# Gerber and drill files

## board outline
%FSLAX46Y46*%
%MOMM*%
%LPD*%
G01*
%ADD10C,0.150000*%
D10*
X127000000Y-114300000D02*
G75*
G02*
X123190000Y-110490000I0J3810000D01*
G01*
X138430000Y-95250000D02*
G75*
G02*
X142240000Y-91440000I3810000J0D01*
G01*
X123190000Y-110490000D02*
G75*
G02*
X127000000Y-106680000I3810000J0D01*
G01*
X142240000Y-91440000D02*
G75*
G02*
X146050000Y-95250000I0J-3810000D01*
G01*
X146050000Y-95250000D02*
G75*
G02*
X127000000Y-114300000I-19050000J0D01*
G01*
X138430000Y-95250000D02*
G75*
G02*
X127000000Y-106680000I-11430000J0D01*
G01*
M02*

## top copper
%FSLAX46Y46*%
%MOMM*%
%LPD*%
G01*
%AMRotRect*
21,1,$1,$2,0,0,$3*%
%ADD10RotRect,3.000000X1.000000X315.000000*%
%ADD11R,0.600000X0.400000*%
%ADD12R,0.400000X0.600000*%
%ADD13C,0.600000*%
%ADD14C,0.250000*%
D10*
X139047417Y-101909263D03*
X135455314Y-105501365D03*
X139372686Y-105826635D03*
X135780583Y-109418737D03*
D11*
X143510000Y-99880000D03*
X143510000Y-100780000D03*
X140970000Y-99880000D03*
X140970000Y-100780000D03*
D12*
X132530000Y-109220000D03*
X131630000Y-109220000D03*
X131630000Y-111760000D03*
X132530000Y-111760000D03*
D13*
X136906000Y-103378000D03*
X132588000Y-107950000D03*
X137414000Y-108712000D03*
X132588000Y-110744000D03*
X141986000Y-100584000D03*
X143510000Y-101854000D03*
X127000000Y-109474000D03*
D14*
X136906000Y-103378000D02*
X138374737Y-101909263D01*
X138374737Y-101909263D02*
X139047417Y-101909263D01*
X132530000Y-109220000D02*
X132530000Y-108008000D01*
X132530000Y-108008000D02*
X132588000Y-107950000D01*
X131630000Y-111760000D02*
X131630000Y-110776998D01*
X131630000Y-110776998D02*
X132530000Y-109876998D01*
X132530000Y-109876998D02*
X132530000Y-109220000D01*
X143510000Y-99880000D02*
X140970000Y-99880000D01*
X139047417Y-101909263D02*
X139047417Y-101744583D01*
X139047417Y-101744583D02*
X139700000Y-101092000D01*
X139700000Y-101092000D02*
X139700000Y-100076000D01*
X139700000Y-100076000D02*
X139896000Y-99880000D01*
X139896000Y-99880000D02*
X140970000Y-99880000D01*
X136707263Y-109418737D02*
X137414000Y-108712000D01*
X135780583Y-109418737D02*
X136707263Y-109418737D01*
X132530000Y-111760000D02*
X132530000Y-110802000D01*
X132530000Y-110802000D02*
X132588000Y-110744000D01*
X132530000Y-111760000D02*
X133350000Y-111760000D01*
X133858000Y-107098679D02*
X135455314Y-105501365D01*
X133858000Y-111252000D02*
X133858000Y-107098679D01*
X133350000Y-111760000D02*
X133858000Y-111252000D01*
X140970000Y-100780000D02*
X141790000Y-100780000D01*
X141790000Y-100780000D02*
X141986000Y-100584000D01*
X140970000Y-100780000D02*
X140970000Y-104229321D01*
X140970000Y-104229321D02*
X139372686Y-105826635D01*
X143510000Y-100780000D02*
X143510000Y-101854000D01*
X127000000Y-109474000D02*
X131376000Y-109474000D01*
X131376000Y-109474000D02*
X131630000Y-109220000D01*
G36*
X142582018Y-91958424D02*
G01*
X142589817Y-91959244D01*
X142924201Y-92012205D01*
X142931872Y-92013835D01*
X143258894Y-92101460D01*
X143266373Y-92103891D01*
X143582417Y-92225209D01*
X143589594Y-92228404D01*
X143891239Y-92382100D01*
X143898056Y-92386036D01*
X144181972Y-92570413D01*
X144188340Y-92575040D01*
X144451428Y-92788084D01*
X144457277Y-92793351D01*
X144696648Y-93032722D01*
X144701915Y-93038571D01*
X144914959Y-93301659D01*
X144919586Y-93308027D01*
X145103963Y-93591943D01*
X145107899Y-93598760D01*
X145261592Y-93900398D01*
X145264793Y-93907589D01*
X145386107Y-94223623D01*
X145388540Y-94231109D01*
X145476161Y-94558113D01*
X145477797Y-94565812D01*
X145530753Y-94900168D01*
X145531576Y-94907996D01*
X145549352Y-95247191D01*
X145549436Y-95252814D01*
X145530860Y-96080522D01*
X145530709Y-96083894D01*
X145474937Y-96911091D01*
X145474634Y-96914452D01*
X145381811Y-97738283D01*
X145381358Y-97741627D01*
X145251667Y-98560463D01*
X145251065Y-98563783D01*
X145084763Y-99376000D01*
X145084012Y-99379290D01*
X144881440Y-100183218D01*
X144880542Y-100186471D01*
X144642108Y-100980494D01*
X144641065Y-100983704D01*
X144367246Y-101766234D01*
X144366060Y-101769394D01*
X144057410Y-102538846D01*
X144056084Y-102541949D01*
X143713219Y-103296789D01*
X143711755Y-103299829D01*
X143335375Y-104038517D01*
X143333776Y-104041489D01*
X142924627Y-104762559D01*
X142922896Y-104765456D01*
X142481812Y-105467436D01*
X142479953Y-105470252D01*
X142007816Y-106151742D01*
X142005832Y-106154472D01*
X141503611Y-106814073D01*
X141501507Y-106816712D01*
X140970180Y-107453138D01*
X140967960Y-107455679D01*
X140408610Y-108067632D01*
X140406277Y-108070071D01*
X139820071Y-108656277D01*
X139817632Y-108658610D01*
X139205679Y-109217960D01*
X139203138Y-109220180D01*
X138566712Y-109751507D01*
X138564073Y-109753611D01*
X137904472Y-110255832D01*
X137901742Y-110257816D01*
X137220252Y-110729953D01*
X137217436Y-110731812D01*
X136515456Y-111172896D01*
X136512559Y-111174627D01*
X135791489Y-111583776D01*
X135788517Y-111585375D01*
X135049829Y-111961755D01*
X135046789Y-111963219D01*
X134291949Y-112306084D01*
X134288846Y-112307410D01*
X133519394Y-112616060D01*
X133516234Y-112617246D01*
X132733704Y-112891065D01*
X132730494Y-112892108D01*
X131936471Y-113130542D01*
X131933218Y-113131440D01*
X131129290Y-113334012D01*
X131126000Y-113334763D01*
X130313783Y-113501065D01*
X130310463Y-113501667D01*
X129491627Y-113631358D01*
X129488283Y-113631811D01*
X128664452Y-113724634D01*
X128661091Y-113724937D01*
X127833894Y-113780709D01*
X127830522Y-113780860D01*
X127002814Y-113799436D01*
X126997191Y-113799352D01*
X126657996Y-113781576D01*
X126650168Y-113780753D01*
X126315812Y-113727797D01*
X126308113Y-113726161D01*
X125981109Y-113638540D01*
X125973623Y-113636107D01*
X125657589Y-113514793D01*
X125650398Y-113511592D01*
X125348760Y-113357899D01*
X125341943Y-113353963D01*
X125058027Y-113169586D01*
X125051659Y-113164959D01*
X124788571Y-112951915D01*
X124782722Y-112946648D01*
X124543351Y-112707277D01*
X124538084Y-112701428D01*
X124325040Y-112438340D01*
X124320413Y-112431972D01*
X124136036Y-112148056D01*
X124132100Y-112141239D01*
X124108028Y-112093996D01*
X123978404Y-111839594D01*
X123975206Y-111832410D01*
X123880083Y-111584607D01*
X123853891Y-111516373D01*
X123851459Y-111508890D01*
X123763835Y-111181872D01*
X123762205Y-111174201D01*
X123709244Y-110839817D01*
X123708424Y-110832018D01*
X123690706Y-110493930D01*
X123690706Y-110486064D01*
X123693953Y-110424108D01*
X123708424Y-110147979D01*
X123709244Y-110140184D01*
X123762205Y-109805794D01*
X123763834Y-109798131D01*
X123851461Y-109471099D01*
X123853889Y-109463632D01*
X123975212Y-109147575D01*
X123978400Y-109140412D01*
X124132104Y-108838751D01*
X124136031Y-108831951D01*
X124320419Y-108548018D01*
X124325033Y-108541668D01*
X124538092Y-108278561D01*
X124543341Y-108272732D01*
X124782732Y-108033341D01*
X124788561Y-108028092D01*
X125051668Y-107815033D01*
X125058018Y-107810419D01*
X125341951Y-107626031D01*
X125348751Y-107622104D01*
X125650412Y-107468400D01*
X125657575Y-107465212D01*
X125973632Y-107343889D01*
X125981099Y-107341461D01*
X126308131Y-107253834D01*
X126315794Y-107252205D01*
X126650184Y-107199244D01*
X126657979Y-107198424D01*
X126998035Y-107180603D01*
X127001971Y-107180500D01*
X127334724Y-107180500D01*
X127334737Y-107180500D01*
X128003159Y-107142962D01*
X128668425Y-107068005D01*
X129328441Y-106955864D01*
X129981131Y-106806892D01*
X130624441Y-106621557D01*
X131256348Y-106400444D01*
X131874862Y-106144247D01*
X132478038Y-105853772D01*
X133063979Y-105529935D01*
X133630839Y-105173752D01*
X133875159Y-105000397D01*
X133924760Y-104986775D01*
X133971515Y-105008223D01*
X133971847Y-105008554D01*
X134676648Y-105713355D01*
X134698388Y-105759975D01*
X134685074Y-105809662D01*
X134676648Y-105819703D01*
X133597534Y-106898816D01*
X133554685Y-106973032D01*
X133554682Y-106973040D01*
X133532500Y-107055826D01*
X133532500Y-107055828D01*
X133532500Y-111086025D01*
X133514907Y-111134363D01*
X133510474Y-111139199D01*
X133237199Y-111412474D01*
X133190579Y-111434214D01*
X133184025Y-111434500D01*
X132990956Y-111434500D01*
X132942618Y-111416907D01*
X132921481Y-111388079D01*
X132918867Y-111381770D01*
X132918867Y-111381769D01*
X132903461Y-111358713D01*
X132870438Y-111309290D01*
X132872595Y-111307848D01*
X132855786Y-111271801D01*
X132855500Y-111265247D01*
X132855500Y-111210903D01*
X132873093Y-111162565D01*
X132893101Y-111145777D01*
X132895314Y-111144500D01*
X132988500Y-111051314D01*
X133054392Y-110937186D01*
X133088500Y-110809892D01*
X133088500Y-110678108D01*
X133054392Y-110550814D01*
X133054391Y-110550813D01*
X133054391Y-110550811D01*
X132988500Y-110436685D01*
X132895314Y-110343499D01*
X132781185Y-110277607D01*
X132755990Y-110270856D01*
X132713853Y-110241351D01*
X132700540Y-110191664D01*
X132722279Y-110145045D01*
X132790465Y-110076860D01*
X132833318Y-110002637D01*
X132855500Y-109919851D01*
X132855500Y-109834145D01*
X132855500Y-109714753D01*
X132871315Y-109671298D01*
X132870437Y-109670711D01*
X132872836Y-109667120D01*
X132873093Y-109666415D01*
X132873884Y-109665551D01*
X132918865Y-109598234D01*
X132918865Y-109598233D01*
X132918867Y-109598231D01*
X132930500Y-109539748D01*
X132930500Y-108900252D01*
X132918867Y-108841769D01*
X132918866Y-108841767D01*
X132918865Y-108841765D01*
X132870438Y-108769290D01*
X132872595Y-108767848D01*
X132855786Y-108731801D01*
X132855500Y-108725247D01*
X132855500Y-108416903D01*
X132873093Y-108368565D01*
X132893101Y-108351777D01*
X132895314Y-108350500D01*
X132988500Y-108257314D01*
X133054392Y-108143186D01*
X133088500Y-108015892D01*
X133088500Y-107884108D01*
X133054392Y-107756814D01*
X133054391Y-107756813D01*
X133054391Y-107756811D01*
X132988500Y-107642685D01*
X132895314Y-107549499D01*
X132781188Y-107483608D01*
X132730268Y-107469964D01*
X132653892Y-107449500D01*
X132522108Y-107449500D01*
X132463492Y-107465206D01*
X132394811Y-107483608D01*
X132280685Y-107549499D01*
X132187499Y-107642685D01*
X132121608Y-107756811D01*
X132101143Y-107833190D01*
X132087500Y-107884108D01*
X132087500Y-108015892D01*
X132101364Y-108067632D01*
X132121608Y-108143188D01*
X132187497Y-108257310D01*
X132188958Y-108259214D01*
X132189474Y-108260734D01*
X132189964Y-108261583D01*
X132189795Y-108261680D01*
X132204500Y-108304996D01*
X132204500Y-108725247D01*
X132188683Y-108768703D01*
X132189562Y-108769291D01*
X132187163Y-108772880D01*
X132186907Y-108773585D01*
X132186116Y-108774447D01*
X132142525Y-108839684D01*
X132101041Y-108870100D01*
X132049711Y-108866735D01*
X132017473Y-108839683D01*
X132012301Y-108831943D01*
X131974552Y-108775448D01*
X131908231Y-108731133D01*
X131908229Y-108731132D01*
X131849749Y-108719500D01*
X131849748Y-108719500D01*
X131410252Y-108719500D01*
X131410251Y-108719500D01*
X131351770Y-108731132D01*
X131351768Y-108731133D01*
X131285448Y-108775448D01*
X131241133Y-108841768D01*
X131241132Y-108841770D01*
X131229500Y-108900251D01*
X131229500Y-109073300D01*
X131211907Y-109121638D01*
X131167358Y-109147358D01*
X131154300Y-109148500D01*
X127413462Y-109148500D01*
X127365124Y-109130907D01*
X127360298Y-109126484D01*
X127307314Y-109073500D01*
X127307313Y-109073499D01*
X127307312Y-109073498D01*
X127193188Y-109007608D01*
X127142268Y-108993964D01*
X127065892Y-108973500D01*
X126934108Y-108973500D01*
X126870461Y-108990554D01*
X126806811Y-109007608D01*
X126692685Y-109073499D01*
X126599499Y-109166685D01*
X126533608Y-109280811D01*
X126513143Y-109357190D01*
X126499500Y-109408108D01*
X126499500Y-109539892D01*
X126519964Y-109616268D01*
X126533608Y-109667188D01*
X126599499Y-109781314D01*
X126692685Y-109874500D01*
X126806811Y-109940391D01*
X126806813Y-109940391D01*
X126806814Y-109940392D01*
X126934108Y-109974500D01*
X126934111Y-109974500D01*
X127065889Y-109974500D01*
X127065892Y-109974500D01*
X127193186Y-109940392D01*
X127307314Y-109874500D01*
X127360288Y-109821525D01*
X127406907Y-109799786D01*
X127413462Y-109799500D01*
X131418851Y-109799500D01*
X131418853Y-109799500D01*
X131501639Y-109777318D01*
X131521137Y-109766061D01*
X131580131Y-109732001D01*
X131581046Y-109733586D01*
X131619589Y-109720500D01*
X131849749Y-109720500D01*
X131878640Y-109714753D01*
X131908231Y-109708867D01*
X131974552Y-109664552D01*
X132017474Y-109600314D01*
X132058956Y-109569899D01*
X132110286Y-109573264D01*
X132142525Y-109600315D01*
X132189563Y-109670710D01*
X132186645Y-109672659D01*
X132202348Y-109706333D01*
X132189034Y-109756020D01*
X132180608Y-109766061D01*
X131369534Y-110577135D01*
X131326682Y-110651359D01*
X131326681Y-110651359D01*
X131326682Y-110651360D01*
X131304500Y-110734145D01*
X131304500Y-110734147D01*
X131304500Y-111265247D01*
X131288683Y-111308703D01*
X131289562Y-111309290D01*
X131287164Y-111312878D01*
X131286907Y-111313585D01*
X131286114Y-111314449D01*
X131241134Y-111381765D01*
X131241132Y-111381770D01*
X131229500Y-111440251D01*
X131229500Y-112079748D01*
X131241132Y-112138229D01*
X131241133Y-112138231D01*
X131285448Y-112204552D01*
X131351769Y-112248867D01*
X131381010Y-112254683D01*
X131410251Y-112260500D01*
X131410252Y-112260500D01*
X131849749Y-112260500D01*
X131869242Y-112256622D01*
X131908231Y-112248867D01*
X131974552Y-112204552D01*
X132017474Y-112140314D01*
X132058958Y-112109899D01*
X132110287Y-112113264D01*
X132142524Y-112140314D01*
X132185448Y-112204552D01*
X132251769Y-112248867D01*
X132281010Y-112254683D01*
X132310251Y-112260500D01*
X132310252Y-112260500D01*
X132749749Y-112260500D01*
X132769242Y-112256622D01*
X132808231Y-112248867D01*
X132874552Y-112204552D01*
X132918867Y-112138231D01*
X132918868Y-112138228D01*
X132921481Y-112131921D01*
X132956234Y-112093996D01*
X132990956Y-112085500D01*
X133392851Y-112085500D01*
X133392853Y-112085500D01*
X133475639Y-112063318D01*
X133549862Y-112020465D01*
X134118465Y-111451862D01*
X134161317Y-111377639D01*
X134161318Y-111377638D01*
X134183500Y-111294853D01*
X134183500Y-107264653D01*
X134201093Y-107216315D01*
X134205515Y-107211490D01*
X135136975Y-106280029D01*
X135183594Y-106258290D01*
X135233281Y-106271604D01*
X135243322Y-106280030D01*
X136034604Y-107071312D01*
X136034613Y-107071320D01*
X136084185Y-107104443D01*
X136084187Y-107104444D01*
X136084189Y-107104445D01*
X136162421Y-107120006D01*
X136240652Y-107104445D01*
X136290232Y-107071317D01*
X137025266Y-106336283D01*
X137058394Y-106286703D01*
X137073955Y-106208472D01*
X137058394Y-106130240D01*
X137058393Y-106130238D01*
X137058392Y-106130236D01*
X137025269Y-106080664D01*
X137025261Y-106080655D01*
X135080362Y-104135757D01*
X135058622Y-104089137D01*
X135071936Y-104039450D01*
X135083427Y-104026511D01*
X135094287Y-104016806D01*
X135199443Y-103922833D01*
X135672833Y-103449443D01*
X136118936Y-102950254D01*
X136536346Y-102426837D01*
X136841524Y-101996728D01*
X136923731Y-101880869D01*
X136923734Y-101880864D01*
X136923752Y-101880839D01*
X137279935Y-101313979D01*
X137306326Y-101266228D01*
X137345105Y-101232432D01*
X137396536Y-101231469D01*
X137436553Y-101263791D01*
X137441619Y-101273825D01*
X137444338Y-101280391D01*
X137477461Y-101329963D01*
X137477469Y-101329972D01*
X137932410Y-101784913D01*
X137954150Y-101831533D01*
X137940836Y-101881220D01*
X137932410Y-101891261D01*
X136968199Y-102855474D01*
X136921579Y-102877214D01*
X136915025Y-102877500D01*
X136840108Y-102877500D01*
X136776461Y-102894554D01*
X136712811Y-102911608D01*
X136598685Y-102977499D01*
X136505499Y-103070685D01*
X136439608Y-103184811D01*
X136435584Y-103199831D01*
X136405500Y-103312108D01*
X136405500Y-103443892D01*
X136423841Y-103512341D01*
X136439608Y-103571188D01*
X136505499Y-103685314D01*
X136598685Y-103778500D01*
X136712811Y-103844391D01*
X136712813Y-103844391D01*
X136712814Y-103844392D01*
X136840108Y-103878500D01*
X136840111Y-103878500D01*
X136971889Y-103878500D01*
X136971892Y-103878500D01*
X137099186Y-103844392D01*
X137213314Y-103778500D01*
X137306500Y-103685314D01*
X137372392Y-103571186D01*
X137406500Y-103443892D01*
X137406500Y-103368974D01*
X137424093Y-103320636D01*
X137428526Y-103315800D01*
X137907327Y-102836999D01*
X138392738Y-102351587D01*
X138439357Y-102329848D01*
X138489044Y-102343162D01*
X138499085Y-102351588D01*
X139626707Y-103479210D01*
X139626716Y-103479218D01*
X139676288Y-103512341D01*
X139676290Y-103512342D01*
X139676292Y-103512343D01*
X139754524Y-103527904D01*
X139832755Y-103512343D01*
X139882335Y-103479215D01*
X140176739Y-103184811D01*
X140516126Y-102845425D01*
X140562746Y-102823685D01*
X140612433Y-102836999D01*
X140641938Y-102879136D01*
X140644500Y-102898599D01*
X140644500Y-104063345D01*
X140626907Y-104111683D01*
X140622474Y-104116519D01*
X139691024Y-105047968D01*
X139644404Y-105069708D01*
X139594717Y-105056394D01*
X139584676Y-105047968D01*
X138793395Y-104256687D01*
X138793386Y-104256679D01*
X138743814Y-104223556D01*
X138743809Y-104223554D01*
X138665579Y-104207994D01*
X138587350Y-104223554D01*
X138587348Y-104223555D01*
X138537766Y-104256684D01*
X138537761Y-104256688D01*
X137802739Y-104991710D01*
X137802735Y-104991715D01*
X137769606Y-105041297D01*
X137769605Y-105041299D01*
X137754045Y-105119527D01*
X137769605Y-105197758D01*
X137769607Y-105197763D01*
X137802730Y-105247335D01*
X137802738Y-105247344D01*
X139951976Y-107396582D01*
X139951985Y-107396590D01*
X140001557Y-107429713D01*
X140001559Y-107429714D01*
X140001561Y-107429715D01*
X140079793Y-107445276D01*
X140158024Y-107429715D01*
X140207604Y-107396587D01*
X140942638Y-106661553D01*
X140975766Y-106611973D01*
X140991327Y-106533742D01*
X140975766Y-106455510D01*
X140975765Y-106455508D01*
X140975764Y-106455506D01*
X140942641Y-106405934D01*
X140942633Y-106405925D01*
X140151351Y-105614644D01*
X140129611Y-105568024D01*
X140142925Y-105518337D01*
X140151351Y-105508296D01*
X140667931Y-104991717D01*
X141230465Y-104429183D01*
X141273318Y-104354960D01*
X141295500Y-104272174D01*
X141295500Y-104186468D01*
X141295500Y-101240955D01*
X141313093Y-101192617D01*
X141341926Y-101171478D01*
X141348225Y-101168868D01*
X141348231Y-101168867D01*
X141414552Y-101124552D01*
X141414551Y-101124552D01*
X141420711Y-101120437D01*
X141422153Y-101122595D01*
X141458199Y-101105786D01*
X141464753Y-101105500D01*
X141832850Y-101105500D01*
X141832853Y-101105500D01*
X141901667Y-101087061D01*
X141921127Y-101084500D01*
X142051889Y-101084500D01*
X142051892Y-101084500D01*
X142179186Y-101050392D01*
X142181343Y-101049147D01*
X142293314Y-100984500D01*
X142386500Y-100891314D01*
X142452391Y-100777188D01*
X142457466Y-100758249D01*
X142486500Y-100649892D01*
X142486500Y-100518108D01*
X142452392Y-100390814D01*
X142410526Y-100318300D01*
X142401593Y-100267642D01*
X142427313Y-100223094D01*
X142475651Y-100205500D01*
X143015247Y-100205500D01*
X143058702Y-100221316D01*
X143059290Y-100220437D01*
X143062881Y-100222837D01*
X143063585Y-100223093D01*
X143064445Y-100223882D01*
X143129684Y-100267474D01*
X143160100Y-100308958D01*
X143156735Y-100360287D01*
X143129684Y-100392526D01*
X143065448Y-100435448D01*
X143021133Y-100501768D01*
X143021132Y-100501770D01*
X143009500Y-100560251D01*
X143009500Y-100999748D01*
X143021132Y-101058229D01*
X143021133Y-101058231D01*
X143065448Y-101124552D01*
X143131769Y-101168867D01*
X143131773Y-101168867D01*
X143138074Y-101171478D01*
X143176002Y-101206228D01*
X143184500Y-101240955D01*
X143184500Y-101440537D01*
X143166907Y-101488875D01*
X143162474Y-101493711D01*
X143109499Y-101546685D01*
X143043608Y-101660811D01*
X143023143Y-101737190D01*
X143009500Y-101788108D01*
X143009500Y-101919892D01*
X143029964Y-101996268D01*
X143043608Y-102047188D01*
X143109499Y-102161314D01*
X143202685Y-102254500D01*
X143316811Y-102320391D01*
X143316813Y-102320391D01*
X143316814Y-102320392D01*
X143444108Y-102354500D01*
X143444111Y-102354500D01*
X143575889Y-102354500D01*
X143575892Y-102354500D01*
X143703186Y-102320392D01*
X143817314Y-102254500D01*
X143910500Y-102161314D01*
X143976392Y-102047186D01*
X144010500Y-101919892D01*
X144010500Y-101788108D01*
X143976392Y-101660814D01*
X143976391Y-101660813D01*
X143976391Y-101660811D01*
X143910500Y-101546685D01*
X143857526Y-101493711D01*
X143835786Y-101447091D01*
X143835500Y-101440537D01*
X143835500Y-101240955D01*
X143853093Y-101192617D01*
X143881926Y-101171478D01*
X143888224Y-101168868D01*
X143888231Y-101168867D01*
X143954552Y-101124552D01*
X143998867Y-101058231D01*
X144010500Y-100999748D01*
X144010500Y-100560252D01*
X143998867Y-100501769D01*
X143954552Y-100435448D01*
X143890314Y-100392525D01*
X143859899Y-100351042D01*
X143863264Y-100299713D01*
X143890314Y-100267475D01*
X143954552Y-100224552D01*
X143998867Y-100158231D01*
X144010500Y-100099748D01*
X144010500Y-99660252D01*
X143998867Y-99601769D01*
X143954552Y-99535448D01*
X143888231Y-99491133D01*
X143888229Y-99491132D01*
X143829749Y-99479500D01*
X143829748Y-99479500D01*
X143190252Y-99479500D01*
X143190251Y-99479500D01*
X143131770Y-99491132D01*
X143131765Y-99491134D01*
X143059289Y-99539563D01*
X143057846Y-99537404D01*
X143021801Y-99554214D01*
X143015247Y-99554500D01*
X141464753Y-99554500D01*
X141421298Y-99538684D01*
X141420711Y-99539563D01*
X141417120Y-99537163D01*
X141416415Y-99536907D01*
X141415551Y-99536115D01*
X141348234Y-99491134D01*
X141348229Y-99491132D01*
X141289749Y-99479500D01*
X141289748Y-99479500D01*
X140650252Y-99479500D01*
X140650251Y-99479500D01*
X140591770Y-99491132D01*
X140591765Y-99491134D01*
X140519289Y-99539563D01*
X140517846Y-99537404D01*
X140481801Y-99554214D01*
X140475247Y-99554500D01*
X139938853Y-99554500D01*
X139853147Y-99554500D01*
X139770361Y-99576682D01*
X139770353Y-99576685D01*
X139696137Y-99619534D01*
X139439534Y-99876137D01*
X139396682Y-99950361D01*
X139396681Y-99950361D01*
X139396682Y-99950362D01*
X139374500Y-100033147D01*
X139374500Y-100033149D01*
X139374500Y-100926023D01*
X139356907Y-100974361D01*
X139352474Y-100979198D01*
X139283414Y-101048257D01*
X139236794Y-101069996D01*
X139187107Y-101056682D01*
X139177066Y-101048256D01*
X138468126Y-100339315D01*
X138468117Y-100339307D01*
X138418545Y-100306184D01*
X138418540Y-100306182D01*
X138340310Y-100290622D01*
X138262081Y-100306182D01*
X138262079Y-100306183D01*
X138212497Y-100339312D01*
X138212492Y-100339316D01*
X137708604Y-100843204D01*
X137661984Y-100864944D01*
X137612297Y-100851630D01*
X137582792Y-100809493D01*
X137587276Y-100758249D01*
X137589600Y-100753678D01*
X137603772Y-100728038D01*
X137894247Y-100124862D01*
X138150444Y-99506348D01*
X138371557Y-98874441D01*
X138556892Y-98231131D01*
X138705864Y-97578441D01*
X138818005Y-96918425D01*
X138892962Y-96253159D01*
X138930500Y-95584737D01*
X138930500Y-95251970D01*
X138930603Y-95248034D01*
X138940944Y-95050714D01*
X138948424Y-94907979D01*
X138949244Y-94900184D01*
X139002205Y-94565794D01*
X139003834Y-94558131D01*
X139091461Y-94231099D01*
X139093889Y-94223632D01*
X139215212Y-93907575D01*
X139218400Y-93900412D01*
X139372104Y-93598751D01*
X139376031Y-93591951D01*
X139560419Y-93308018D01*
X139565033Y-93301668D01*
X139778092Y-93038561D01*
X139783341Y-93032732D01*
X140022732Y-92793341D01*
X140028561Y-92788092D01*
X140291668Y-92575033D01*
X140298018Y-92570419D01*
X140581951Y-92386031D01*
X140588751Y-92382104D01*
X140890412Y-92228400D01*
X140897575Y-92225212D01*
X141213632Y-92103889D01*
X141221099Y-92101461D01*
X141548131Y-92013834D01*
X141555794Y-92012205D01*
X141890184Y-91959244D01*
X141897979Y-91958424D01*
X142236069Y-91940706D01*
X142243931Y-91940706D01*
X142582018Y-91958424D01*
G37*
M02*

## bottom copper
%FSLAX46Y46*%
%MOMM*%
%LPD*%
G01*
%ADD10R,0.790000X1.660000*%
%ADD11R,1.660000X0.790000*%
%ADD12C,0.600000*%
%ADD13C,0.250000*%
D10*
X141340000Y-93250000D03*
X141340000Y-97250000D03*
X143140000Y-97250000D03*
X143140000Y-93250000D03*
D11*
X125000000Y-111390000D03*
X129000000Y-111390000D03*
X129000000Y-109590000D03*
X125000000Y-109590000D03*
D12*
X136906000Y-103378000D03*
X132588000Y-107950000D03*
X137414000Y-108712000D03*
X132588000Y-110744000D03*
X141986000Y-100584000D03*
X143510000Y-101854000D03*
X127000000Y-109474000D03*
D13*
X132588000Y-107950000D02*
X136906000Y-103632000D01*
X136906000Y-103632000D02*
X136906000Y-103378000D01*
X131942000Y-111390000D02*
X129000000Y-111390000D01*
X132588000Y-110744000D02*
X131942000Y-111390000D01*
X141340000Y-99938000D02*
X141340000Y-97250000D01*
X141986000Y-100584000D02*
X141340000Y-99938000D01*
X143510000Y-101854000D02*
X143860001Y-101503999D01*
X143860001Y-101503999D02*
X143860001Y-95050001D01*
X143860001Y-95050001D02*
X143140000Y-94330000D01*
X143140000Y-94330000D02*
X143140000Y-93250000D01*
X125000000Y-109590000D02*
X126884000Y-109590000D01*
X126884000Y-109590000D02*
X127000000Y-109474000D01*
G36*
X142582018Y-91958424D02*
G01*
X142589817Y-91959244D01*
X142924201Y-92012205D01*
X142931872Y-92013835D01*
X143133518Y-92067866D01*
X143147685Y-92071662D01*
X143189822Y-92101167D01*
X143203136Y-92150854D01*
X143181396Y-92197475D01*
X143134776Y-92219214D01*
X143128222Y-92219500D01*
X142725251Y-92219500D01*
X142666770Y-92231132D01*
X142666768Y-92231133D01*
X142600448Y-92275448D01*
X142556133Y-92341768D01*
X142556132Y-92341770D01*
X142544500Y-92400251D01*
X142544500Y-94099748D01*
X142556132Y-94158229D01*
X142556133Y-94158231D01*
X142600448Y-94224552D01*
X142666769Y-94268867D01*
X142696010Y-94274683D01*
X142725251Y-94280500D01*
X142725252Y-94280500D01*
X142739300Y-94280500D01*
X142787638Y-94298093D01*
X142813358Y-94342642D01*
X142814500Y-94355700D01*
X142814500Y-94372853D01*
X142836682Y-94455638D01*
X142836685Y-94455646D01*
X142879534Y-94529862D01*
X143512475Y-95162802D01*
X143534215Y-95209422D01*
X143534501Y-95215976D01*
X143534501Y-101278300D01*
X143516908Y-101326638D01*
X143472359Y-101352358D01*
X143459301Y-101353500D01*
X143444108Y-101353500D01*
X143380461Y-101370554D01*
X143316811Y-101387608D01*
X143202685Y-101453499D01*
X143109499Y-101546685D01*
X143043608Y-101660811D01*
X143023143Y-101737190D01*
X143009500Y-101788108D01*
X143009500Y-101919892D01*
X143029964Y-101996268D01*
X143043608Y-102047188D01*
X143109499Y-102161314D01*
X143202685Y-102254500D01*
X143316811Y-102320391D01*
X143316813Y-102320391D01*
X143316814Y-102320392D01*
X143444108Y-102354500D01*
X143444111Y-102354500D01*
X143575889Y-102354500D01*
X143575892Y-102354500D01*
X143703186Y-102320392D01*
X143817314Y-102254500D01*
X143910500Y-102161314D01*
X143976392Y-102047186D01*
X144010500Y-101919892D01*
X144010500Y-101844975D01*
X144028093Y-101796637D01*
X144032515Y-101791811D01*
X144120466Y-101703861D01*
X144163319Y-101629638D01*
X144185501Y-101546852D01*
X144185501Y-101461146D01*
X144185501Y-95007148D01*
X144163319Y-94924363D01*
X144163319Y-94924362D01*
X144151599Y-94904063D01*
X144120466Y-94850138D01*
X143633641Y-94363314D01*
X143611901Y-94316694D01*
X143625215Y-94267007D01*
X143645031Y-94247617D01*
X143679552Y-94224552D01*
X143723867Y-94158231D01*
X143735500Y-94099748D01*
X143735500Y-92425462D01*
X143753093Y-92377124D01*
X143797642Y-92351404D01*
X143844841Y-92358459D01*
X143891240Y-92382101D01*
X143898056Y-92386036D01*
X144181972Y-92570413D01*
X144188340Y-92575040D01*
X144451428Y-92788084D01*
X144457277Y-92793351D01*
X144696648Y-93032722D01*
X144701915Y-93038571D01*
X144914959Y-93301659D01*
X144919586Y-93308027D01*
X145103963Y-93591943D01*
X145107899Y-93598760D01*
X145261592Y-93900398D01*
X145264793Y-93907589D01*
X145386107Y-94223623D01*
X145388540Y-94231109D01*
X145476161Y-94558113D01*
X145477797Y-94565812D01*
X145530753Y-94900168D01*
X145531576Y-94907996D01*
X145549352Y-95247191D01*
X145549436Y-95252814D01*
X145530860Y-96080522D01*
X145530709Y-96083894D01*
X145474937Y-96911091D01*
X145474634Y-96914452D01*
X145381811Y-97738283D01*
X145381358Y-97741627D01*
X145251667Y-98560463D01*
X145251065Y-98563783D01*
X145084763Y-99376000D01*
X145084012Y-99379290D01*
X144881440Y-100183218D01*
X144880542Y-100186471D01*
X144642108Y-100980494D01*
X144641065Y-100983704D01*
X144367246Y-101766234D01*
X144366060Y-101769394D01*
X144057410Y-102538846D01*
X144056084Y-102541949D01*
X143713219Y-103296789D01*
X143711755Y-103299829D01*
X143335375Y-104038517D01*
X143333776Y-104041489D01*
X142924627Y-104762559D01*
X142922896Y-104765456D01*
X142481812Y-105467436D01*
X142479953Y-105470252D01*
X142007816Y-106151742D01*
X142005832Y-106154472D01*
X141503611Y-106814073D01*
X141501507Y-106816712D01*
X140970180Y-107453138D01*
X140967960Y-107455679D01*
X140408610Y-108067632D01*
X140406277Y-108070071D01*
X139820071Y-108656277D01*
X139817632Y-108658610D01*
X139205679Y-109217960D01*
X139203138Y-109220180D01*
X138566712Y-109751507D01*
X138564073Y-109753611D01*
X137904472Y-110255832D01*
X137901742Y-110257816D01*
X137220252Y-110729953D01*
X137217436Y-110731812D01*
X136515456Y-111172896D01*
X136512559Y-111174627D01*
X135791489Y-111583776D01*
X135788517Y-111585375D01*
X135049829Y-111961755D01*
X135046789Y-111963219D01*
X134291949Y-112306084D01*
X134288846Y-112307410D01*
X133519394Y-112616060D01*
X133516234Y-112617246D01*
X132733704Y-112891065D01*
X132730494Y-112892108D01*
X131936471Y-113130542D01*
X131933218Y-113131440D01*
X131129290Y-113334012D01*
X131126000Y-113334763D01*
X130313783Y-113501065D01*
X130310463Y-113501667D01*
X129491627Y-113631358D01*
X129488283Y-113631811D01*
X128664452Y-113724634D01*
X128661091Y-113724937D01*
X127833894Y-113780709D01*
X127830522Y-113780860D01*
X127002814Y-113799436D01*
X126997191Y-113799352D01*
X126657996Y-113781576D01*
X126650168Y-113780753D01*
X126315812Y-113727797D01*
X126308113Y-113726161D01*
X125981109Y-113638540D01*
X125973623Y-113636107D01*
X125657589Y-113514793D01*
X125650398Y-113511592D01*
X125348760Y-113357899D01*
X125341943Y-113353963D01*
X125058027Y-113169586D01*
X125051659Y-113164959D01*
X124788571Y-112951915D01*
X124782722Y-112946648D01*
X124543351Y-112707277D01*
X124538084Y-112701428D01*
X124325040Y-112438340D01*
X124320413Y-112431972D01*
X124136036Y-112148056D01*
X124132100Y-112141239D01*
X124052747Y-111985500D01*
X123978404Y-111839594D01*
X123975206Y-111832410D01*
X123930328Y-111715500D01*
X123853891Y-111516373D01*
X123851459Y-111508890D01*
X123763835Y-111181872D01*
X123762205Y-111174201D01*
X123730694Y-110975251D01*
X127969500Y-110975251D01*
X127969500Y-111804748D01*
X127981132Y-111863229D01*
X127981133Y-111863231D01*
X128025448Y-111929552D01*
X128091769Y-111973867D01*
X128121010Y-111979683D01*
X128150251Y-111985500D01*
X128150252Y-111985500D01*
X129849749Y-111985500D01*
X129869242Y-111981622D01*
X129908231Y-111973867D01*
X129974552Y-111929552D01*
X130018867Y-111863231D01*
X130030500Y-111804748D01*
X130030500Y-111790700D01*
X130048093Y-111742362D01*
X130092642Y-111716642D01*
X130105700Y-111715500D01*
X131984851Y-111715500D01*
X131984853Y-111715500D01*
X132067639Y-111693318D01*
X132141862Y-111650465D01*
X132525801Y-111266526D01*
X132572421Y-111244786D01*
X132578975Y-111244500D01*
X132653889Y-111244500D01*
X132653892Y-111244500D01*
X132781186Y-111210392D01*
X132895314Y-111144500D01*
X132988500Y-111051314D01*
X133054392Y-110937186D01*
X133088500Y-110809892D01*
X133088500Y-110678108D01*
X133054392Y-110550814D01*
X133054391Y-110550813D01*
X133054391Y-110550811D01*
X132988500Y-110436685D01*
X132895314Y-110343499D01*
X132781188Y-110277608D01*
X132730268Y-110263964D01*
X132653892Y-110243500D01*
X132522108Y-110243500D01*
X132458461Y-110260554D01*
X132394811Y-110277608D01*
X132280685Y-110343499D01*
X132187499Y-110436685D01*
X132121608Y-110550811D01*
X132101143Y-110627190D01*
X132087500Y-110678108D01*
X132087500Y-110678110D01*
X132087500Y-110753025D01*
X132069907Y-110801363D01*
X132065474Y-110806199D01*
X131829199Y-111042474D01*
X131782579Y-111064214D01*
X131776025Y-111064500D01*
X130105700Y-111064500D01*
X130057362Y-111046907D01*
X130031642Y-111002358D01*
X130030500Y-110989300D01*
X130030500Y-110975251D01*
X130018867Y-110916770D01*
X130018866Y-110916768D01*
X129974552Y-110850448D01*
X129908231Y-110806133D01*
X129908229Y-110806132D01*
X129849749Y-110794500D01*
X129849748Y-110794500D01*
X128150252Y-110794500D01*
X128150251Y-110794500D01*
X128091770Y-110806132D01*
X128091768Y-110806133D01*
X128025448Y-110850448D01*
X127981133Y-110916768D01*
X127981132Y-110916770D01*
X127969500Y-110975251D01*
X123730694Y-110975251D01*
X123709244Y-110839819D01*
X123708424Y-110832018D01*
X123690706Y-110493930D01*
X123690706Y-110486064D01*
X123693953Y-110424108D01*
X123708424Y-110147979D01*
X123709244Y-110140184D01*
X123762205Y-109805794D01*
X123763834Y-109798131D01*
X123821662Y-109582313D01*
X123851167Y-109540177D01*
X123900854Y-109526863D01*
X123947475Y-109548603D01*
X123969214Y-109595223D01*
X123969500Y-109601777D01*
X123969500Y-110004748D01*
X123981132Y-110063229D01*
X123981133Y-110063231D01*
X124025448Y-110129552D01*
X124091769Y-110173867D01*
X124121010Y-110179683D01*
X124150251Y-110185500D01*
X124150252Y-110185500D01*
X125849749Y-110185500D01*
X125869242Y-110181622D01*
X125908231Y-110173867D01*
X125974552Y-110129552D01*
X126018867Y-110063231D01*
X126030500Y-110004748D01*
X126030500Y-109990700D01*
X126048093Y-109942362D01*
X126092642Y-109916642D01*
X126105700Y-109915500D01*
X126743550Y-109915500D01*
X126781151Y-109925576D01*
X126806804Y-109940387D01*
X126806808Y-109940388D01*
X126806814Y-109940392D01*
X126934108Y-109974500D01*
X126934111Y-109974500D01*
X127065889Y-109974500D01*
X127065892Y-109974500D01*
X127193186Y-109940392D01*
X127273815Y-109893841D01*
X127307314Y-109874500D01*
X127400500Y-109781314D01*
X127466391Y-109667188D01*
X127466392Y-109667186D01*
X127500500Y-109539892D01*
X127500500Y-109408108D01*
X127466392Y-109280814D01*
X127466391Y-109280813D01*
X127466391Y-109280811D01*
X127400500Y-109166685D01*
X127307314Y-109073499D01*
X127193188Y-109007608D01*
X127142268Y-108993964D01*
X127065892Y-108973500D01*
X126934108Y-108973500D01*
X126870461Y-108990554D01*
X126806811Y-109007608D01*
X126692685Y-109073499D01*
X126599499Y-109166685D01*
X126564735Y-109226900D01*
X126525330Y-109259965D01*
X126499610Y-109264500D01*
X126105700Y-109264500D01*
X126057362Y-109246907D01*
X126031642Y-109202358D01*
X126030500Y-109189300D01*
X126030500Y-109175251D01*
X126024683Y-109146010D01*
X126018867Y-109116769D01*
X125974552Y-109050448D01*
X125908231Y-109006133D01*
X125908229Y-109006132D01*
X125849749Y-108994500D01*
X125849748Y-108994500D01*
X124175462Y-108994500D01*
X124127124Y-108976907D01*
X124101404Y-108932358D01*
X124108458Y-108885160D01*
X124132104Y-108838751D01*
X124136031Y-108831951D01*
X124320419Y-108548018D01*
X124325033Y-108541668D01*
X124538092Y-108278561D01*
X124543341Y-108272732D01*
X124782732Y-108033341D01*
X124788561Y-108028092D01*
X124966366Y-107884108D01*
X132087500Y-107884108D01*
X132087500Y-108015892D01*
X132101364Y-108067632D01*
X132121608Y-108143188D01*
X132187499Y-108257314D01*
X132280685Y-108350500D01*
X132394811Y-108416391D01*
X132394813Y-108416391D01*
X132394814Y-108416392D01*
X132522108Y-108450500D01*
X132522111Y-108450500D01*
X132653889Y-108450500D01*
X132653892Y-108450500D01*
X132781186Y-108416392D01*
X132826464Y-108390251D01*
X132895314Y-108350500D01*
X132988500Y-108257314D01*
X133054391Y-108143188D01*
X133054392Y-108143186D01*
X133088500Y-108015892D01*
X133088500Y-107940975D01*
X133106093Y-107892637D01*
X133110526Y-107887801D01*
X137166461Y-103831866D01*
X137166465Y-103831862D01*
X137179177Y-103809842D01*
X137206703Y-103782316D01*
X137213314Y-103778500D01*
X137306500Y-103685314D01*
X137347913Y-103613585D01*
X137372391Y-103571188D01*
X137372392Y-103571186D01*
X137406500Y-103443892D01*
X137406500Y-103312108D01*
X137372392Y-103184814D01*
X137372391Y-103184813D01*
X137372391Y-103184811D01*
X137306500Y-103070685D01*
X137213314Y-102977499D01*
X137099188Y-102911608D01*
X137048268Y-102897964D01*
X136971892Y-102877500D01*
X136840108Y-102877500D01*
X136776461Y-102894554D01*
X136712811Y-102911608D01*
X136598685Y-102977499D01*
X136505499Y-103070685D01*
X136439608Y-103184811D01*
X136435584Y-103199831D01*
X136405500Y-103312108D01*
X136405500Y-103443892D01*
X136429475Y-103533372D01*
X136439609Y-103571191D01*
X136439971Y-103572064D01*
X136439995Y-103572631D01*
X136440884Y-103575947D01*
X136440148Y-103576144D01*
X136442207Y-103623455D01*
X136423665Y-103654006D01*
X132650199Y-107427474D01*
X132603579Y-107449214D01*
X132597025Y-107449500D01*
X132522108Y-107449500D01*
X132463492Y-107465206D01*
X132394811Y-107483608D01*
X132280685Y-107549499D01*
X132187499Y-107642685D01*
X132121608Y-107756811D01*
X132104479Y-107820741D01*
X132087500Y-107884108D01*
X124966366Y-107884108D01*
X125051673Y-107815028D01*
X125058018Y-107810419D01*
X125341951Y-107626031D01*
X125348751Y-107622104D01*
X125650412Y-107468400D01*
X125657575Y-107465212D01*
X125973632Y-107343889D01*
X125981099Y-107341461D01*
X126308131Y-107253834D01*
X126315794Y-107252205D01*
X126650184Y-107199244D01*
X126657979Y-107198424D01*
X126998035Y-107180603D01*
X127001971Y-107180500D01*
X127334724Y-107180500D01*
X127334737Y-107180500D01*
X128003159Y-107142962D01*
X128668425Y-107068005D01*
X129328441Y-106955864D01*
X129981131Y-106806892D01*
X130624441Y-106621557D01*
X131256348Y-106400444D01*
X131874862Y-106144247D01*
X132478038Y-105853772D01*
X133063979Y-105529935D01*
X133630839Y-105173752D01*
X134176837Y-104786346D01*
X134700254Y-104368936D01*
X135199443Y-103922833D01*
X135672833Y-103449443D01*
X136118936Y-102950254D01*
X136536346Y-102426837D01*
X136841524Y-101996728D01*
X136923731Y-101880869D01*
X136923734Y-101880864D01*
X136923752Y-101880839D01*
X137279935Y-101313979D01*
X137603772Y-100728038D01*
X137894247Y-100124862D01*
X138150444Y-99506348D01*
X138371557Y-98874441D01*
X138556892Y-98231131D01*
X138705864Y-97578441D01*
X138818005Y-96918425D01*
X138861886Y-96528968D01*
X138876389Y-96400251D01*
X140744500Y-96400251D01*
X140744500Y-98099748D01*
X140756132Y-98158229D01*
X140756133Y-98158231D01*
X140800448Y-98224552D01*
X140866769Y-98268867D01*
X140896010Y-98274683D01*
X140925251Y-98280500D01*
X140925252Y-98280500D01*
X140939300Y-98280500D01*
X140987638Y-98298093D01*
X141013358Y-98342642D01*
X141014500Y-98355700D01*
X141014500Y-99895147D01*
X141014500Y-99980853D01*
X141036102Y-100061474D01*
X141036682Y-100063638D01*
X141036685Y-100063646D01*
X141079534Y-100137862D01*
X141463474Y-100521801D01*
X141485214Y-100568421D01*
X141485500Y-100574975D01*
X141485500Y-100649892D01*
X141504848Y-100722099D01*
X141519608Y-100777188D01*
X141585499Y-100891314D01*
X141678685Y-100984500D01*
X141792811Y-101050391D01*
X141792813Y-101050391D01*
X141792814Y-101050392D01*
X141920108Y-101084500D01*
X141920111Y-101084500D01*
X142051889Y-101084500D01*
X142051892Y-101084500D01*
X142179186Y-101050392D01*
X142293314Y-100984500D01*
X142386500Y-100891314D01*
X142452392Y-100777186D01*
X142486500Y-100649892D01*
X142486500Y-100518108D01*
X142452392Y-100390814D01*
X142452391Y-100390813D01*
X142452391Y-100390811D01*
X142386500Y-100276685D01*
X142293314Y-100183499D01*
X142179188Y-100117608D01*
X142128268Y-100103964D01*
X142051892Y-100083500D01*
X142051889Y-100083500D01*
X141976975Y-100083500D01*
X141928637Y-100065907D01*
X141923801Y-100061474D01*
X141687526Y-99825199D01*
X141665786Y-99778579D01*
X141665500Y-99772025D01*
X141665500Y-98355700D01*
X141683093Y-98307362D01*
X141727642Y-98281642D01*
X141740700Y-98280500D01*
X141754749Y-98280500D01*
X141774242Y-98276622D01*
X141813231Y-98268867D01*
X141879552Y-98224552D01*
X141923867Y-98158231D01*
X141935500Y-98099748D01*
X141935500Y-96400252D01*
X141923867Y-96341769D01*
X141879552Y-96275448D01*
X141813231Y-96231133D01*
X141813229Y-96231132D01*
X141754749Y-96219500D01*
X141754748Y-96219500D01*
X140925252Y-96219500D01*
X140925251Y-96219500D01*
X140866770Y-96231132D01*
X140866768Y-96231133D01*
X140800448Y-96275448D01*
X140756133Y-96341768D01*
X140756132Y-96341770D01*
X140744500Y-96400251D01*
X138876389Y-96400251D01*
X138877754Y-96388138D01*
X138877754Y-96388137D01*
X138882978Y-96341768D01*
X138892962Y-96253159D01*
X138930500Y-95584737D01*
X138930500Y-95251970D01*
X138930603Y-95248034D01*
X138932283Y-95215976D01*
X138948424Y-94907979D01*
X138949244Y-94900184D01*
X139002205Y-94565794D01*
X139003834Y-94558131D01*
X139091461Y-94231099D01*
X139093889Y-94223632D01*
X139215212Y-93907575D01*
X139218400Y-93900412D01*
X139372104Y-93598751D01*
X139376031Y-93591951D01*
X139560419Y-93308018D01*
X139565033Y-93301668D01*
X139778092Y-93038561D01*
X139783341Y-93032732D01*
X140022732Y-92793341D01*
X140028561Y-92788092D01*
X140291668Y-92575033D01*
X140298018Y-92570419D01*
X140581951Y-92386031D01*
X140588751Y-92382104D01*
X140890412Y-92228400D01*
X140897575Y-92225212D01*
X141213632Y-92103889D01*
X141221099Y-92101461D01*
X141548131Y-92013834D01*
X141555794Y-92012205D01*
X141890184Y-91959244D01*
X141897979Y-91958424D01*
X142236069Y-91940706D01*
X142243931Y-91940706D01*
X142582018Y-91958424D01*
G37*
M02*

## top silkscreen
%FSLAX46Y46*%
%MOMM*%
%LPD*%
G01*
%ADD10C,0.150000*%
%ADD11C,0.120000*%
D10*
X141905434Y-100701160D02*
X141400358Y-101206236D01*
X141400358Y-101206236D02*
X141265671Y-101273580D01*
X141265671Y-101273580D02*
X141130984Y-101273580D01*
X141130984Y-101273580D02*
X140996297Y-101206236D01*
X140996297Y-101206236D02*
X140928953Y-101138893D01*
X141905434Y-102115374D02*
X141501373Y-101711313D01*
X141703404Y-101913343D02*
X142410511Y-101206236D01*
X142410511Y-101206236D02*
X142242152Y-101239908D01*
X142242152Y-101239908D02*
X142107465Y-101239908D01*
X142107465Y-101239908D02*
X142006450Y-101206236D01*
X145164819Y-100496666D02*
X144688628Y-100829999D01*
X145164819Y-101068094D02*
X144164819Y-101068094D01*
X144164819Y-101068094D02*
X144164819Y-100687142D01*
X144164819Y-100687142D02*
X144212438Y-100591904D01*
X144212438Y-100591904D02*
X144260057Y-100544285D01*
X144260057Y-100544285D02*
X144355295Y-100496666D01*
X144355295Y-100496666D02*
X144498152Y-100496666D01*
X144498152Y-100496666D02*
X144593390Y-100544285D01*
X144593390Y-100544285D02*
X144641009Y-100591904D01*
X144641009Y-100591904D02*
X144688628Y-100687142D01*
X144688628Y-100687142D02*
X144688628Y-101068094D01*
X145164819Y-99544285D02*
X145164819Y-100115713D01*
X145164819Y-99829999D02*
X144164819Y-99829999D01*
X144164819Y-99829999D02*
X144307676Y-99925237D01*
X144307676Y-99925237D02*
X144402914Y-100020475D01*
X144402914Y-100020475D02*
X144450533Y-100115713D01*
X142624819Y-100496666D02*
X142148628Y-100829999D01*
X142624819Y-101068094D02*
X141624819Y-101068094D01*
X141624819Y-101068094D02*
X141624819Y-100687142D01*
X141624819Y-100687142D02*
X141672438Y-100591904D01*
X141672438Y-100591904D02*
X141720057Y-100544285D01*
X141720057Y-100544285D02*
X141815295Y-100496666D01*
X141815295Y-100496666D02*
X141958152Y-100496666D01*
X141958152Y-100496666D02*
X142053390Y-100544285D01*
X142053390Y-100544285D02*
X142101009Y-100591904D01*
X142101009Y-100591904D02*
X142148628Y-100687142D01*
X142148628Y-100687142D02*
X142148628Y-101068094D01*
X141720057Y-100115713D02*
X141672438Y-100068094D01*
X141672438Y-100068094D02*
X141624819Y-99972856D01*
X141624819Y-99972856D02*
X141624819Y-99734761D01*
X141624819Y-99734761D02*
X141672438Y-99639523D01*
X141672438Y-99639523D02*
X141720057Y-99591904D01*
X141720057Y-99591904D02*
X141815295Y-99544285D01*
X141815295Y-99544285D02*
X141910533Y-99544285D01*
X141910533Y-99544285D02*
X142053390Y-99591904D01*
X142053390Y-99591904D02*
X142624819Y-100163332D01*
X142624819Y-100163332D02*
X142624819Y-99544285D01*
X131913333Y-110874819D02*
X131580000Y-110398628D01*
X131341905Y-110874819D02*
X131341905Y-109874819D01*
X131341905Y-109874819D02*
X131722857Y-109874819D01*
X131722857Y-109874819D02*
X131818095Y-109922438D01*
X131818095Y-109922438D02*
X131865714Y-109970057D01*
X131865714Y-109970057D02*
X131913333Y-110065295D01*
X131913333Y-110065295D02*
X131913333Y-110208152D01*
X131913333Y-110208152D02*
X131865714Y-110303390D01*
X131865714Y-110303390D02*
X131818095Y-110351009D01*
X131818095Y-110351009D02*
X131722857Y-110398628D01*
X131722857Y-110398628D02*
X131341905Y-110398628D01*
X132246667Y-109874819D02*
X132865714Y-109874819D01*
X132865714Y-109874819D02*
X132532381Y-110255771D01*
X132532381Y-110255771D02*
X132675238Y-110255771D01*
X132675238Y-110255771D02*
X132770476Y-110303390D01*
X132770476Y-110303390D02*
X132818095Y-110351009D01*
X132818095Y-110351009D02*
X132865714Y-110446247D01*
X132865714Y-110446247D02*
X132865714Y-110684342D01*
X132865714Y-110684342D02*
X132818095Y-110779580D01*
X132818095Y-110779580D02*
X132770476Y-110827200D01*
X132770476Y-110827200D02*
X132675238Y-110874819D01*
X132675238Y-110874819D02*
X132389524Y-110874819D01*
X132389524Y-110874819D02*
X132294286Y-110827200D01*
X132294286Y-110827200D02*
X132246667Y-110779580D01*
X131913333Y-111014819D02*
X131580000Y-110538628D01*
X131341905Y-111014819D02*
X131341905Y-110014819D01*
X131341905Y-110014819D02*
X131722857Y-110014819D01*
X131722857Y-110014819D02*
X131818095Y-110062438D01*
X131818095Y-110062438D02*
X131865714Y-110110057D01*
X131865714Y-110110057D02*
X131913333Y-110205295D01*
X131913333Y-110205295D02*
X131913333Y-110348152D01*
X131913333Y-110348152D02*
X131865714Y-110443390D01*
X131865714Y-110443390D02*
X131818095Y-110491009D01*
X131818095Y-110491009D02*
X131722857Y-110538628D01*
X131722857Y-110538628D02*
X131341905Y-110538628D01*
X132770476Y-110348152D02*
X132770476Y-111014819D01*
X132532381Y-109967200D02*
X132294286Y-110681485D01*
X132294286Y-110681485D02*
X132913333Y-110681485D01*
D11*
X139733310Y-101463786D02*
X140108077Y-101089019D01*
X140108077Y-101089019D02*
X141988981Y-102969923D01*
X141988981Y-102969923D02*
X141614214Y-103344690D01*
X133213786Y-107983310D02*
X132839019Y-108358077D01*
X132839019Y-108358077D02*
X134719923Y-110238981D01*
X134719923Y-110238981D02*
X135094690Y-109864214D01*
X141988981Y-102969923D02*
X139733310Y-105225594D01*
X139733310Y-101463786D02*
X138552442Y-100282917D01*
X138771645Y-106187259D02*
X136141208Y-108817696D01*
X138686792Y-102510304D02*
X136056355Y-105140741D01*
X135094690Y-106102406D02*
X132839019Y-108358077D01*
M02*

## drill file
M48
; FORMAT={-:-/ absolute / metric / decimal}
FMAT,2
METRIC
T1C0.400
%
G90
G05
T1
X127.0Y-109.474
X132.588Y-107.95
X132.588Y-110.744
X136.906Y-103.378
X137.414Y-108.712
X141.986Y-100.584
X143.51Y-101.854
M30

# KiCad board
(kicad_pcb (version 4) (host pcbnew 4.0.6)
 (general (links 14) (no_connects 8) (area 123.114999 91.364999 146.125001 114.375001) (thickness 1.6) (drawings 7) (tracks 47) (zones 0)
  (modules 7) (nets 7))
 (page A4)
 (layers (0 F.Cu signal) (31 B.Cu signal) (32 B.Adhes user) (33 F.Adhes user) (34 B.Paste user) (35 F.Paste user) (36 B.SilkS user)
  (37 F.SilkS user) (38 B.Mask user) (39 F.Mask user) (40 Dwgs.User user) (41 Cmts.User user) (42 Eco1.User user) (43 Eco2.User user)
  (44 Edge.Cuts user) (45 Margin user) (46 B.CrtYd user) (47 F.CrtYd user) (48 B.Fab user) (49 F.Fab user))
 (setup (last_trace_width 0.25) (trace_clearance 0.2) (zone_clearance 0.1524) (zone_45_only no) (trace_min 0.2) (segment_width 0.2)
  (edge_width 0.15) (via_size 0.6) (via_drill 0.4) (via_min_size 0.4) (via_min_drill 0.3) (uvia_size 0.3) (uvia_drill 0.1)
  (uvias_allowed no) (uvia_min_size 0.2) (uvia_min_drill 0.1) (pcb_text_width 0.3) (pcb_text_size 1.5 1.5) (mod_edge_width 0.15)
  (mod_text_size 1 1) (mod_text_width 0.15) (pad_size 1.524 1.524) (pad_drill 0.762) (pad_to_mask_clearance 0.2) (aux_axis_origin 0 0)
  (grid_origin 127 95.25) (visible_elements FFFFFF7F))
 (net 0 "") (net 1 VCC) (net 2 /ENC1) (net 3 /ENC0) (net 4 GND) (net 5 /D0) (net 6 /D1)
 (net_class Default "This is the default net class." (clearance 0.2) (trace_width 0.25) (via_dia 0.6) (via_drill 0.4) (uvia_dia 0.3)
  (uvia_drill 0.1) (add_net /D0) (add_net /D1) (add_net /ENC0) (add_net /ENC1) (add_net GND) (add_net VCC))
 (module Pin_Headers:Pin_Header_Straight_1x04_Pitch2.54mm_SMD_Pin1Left (layer F.Cu) (at 137.414 105.664 315)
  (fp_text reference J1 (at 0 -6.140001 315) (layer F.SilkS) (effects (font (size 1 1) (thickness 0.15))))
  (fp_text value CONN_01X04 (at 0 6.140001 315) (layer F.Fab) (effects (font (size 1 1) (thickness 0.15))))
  (fp_line (start -1.33 -4.61) (end -1.33 -5.14) (layer F.SilkS) (width 0.12))
  (fp_line (start -1.33 -5.14) (end 1.33 -5.14) (layer F.SilkS) (width 0.12))
  (fp_line (start 1.33 -5.14) (end 1.33 -4.61) (layer F.SilkS) (width 0.12))
  (fp_line (start -1.33 4.61) (end -1.33 5.14) (layer F.SilkS) (width 0.12))
  (fp_line (start -1.33 5.14) (end 1.33 5.14) (layer F.SilkS) (width 0.12))
  (fp_line (start 1.33 5.14) (end 1.33 4.61) (layer F.SilkS) (width 0.12))
  (fp_line (start 1.33 -5.14) (end 1.33 -1.95) (layer F.SilkS) (width 0.12))
  (fp_line (start -1.33 -4.61) (end -3 -4.61) (layer F.SilkS) (width 0.12))
  (fp_line (start 1.33 -0.59) (end 1.33 3.13) (layer F.SilkS) (width 0.12))
  (fp_line (start -1.33 -3.13) (end -1.33 0.59) (layer F.SilkS) (width 0.12))
  (fp_line (start -1.33 1.95) (end -1.33 5.14) (layer F.SilkS) (width 0.12))
  (pad 1 smd rect (at -1.5 -3.81 315) (size 3 1) (layers F.Cu F.Paste F.Mask) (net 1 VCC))
  (pad 3 smd rect (at -1.5 1.27 315) (size 3 1) (layers F.Cu F.Paste F.Mask) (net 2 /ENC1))
  (pad 2 smd rect (at 1.5 -1.27 315) (size 3 1) (layers F.Cu F.Paste F.Mask) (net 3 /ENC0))
  (pad 4 smd rect (at 1.5 3.81 315) (size 3 1) (layers F.Cu F.Paste F.Mask) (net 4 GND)))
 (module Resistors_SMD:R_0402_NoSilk (layer F.Cu) (at 143.51 100.33 270)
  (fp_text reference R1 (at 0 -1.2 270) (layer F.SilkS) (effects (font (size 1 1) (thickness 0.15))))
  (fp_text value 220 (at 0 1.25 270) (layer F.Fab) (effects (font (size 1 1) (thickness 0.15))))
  (pad 1 smd rect (at -0.45 0 270) (size 0.4 0.6) (layers F.Cu F.Paste F.Mask) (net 1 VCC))
  (pad 2 smd rect (at 0.45 0 270) (size 0.4 0.6) (layers F.Cu F.Paste F.Mask) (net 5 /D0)))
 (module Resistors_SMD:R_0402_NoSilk (layer F.Cu) (at 140.97 100.33 270)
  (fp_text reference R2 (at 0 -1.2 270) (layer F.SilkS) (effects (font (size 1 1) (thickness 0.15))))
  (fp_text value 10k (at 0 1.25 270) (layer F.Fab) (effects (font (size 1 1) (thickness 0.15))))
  (pad 1 smd rect (at -0.45 0 270) (size 0.4 0.6) (layers F.Cu F.Paste F.Mask) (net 1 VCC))
  (pad 2 smd rect (at 0.45 0 270) (size 0.4 0.6) (layers F.Cu F.Paste F.Mask) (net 3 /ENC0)))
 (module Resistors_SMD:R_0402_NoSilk (layer F.Cu) (at 132.08 109.22 180)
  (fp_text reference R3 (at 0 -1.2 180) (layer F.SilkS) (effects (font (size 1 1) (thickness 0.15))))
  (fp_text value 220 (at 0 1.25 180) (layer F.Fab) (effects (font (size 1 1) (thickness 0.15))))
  (pad 1 smd rect (at -0.45 0 180) (size 0.4 0.6) (layers F.Cu F.Paste F.Mask) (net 1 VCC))
  (pad 2 smd rect (at 0.45 0 180) (size 0.4 0.6) (layers F.Cu F.Paste F.Mask) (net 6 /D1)))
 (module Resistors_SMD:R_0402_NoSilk (layer F.Cu) (at 132.08 111.76)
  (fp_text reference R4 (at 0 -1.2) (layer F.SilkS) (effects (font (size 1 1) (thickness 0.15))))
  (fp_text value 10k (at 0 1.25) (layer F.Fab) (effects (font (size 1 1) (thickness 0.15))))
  (pad 1 smd rect (at -0.45 0) (size 0.4 0.6) (layers F.Cu F.Paste F.Mask) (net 1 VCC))
  (pad 2 smd rect (at 0.45 0) (size 0.4 0.6) (layers F.Cu F.Paste F.Mask) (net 2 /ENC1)))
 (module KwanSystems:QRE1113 (layer B.Cu) (at 142.24 95.25 270)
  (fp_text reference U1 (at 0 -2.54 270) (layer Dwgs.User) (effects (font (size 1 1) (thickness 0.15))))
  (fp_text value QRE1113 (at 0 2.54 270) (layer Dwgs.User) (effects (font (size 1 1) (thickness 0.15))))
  (pad 4 smd rect (at -2 0.9 270) (size 1.66 0.79) (layers B.Cu B.Paste B.Mask) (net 4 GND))
  (pad 3 smd rect (at 2 0.9 270) (size 1.66 0.79) (layers B.Cu B.Paste B.Mask) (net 3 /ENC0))
  (pad 2 smd rect (at 2 -0.9 270) (size 1.66 0.79) (layers B.Cu B.Paste B.Mask) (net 4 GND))
  (pad 1 smd rect (at -2 -0.9 270) (size 1.66 0.79) (layers B.Cu B.Paste B.Mask) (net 5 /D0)))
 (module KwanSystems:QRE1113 (layer B.Cu) (at 127 110.49)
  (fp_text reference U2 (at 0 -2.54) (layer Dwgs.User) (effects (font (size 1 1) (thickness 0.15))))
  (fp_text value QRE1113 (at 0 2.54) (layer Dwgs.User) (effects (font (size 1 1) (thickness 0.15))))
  (pad 4 smd rect (at -2 0.9) (size 1.66 0.79) (layers B.Cu B.Paste B.Mask) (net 4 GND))
  (pad 3 smd rect (at 2 0.9) (size 1.66 0.79) (layers B.Cu B.Paste B.Mask) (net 2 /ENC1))
  (pad 2 smd rect (at 2 -0.9) (size 1.66 0.79) (layers B.Cu B.Paste B.Mask) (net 4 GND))
  (pad 1 smd rect (at -2 -0.9) (size 1.66 0.79) (layers B.Cu B.Paste B.Mask) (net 6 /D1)))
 (gr_arc (start 127 110.49) (end 127 114.3) (angle 90) (layer Edge.Cuts) (width 0.15))
 (gr_arc (start 142.24 95.25) (end 138.43 95.25) (angle 90) (layer Edge.Cuts) (width 0.15))
 (gr_arc (start 127 110.49) (end 123.19 110.49) (angle 90) (layer Edge.Cuts) (width 0.15))
 (gr_arc (start 142.24 95.25) (end 142.24 91.44) (angle 90) (layer Edge.Cuts) (width 0.15))
 (gr_arc (start 127 95.25) (end 146.05 95.25) (angle 90) (layer Edge.Cuts) (width 0.15))
 (gr_arc (start 127 95.25) (end 138.43 95.25) (angle 90) (layer Edge.Cuts) (width 0.15))
 (segment (start 136.906 103.378) (end 138.374737 101.909263) (width 0.25) (layer F.Cu) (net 1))
 (segment (start 138.374737 101.909263) (end 139.047417 101.909263) (width 0.25) (layer F.Cu) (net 1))
 (segment (start 132.588 107.95) (end 136.906 103.632) (width 0.25) (layer B.Cu) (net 1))
 (segment (start 136.906 103.632) (end 136.906 103.378) (width 0.25) (layer B.Cu) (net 1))
 (via (at 136.906 103.378) (size 0.6) (drill 0.4) (layers F.Cu B.Cu) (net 1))
 (segment (start 132.53 109.22) (end 132.53 108.008) (width 0.25) (layer F.Cu) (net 1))
 (segment (start 132.53 108.008) (end 132.588 107.95) (width 0.25) (layer F.Cu) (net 1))
 (via (at 132.588 107.95) (size 0.6) (drill 0.4) (layers F.Cu B.Cu) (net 1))
 (segment (start 131.63 111.76) (end 131.63 110.776998) (width 0.25) (layer F.Cu) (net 1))
 (segment (start 131.63 110.776998) (end 132.53 109.876998) (width 0.25) (layer F.Cu) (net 1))
 (segment (start 132.53 109.876998) (end 132.53 109.22) (width 0.25) (layer F.Cu) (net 1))
 (segment (start 143.51 99.88) (end 140.97 99.88) (width 0.25) (layer F.Cu) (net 1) (status C00000))
 (segment (start 139.047417 101.909263) (end 139.047417 101.744583) (width 0.25) (layer F.Cu) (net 1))
 (segment (start 139.047417 101.744583) (end 139.7 101.092) (width 0.25) (layer F.Cu) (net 1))
 (segment (start 139.7 101.092) (end 139.7 100.076) (width 0.25) (layer F.Cu) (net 1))
 (segment (start 139.7 100.076) (end 139.896 99.88) (width 0.25) (layer F.Cu) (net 1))
 (segment (start 139.896 99.88) (end 140.97 99.88) (width 0.25) (layer F.Cu) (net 1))
 (segment (start 136.707263 109.418737) (end 137.414 108.712) (width 0.25) (layer F.Cu) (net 4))
 (via (at 137.414 108.712) (size 0.6) (drill 0.4) (layers F.Cu B.Cu) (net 4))
 (segment (start 135.780583 109.418737) (end 136.707263 109.418737) (width 0.25) (layer F.Cu) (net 4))
 (segment (start 132.53 111.76) (end 132.53 110.802) (width 0.25) (layer F.Cu) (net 2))
 (segment (start 131.942 111.39) (end 129 111.39) (width 0.25) (layer B.Cu) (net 2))
 (segment (start 132.588 110.744) (end 131.942 111.39) (width 0.25) (layer B.Cu) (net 2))
 (via (at 132.588 110.744) (size 0.6) (drill 0.4) (layers F.Cu B.Cu) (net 2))
 (segment (start 132.53 110.802) (end 132.588 110.744) (width 0.25) (layer F.Cu) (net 2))
 (segment (start 132.53 111.76) (end 133.35 111.76) (width 0.25) (layer F.Cu) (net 2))
 (segment (start 133.858 107.098679) (end 135.455314 105.501365) (width 0.25) (layer F.Cu) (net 2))
 (segment (start 133.858 111.252) (end 133.858 107.098679) (width 0.25) (layer F.Cu) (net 2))
 (segment (start 133.35 111.76) (end 133.858 111.252) (width 0.25) (layer F.Cu) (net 2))
 (segment (start 140.97 100.78) (end 141.79 100.78) (width 0.25) (layer F.Cu) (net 3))
 (segment (start 141.34 99.938) (end 141.34 97.25) (width 0.25) (layer B.Cu) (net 3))
 (segment (start 141.986 100.584) (end 141.34 99.938) (width 0.25) (layer B.Cu) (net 3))
 (via (at 141.986 100.584) (size 0.6) (drill 0.4) (layers F.Cu B.Cu) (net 3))
 (segment (start 141.79 100.78) (end 141.986 100.584) (width 0.25) (layer F.Cu) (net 3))
 (segment (start 140.97 100.78) (end 140.97 104.229321) (width 0.25) (layer F.Cu) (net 3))
 (segment (start 140.97 104.229321) (end 139.372686 105.826635) (width 0.25) (layer F.Cu) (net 3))
 (segment (start 143.51 101.854) (end 143.860001 101.503999) (width 0.25) (layer B.Cu) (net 5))
 (segment (start 143.860001 101.503999) (end 143.860001 95.050001) (width 0.25) (layer B.Cu) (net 5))
 (segment (start 143.860001 95.050001) (end 143.14 94.33) (width 0.25) (layer B.Cu) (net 5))
 (segment (start 143.14 94.33) (end 143.14 93.25) (width 0.25) (layer B.Cu) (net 5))
 (segment (start 143.51 100.78) (end 143.51 101.854) (width 0.25) (layer F.Cu) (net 5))
 (via (at 143.51 101.854) (size 0.6) (drill 0.4) (layers F.Cu B.Cu) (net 5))
 (segment (start 127 109.474) (end 131.376 109.474) (width 0.25) (layer F.Cu) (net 6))
 (segment (start 131.376 109.474) (end 131.63 109.22) (width 0.25) (layer F.Cu) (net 6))
 (segment (start 125 109.59) (end 126.884 109.59) (width 0.25) (layer B.Cu) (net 6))
 (segment (start 126.884 109.59) (end 127 109.474) (width 0.25) (layer B.Cu) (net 6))
 (via (at 127 109.474) (size 0.6) (drill 0.4) (layers F.Cu B.Cu) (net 6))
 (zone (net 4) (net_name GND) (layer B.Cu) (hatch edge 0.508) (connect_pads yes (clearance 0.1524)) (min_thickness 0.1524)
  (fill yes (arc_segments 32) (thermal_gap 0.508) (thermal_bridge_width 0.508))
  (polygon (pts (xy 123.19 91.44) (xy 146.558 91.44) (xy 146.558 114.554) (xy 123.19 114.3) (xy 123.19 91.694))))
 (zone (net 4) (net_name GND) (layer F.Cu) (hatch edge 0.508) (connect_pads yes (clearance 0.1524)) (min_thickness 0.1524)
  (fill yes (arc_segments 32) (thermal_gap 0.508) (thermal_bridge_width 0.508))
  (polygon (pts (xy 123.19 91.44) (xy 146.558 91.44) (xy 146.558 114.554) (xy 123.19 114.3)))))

